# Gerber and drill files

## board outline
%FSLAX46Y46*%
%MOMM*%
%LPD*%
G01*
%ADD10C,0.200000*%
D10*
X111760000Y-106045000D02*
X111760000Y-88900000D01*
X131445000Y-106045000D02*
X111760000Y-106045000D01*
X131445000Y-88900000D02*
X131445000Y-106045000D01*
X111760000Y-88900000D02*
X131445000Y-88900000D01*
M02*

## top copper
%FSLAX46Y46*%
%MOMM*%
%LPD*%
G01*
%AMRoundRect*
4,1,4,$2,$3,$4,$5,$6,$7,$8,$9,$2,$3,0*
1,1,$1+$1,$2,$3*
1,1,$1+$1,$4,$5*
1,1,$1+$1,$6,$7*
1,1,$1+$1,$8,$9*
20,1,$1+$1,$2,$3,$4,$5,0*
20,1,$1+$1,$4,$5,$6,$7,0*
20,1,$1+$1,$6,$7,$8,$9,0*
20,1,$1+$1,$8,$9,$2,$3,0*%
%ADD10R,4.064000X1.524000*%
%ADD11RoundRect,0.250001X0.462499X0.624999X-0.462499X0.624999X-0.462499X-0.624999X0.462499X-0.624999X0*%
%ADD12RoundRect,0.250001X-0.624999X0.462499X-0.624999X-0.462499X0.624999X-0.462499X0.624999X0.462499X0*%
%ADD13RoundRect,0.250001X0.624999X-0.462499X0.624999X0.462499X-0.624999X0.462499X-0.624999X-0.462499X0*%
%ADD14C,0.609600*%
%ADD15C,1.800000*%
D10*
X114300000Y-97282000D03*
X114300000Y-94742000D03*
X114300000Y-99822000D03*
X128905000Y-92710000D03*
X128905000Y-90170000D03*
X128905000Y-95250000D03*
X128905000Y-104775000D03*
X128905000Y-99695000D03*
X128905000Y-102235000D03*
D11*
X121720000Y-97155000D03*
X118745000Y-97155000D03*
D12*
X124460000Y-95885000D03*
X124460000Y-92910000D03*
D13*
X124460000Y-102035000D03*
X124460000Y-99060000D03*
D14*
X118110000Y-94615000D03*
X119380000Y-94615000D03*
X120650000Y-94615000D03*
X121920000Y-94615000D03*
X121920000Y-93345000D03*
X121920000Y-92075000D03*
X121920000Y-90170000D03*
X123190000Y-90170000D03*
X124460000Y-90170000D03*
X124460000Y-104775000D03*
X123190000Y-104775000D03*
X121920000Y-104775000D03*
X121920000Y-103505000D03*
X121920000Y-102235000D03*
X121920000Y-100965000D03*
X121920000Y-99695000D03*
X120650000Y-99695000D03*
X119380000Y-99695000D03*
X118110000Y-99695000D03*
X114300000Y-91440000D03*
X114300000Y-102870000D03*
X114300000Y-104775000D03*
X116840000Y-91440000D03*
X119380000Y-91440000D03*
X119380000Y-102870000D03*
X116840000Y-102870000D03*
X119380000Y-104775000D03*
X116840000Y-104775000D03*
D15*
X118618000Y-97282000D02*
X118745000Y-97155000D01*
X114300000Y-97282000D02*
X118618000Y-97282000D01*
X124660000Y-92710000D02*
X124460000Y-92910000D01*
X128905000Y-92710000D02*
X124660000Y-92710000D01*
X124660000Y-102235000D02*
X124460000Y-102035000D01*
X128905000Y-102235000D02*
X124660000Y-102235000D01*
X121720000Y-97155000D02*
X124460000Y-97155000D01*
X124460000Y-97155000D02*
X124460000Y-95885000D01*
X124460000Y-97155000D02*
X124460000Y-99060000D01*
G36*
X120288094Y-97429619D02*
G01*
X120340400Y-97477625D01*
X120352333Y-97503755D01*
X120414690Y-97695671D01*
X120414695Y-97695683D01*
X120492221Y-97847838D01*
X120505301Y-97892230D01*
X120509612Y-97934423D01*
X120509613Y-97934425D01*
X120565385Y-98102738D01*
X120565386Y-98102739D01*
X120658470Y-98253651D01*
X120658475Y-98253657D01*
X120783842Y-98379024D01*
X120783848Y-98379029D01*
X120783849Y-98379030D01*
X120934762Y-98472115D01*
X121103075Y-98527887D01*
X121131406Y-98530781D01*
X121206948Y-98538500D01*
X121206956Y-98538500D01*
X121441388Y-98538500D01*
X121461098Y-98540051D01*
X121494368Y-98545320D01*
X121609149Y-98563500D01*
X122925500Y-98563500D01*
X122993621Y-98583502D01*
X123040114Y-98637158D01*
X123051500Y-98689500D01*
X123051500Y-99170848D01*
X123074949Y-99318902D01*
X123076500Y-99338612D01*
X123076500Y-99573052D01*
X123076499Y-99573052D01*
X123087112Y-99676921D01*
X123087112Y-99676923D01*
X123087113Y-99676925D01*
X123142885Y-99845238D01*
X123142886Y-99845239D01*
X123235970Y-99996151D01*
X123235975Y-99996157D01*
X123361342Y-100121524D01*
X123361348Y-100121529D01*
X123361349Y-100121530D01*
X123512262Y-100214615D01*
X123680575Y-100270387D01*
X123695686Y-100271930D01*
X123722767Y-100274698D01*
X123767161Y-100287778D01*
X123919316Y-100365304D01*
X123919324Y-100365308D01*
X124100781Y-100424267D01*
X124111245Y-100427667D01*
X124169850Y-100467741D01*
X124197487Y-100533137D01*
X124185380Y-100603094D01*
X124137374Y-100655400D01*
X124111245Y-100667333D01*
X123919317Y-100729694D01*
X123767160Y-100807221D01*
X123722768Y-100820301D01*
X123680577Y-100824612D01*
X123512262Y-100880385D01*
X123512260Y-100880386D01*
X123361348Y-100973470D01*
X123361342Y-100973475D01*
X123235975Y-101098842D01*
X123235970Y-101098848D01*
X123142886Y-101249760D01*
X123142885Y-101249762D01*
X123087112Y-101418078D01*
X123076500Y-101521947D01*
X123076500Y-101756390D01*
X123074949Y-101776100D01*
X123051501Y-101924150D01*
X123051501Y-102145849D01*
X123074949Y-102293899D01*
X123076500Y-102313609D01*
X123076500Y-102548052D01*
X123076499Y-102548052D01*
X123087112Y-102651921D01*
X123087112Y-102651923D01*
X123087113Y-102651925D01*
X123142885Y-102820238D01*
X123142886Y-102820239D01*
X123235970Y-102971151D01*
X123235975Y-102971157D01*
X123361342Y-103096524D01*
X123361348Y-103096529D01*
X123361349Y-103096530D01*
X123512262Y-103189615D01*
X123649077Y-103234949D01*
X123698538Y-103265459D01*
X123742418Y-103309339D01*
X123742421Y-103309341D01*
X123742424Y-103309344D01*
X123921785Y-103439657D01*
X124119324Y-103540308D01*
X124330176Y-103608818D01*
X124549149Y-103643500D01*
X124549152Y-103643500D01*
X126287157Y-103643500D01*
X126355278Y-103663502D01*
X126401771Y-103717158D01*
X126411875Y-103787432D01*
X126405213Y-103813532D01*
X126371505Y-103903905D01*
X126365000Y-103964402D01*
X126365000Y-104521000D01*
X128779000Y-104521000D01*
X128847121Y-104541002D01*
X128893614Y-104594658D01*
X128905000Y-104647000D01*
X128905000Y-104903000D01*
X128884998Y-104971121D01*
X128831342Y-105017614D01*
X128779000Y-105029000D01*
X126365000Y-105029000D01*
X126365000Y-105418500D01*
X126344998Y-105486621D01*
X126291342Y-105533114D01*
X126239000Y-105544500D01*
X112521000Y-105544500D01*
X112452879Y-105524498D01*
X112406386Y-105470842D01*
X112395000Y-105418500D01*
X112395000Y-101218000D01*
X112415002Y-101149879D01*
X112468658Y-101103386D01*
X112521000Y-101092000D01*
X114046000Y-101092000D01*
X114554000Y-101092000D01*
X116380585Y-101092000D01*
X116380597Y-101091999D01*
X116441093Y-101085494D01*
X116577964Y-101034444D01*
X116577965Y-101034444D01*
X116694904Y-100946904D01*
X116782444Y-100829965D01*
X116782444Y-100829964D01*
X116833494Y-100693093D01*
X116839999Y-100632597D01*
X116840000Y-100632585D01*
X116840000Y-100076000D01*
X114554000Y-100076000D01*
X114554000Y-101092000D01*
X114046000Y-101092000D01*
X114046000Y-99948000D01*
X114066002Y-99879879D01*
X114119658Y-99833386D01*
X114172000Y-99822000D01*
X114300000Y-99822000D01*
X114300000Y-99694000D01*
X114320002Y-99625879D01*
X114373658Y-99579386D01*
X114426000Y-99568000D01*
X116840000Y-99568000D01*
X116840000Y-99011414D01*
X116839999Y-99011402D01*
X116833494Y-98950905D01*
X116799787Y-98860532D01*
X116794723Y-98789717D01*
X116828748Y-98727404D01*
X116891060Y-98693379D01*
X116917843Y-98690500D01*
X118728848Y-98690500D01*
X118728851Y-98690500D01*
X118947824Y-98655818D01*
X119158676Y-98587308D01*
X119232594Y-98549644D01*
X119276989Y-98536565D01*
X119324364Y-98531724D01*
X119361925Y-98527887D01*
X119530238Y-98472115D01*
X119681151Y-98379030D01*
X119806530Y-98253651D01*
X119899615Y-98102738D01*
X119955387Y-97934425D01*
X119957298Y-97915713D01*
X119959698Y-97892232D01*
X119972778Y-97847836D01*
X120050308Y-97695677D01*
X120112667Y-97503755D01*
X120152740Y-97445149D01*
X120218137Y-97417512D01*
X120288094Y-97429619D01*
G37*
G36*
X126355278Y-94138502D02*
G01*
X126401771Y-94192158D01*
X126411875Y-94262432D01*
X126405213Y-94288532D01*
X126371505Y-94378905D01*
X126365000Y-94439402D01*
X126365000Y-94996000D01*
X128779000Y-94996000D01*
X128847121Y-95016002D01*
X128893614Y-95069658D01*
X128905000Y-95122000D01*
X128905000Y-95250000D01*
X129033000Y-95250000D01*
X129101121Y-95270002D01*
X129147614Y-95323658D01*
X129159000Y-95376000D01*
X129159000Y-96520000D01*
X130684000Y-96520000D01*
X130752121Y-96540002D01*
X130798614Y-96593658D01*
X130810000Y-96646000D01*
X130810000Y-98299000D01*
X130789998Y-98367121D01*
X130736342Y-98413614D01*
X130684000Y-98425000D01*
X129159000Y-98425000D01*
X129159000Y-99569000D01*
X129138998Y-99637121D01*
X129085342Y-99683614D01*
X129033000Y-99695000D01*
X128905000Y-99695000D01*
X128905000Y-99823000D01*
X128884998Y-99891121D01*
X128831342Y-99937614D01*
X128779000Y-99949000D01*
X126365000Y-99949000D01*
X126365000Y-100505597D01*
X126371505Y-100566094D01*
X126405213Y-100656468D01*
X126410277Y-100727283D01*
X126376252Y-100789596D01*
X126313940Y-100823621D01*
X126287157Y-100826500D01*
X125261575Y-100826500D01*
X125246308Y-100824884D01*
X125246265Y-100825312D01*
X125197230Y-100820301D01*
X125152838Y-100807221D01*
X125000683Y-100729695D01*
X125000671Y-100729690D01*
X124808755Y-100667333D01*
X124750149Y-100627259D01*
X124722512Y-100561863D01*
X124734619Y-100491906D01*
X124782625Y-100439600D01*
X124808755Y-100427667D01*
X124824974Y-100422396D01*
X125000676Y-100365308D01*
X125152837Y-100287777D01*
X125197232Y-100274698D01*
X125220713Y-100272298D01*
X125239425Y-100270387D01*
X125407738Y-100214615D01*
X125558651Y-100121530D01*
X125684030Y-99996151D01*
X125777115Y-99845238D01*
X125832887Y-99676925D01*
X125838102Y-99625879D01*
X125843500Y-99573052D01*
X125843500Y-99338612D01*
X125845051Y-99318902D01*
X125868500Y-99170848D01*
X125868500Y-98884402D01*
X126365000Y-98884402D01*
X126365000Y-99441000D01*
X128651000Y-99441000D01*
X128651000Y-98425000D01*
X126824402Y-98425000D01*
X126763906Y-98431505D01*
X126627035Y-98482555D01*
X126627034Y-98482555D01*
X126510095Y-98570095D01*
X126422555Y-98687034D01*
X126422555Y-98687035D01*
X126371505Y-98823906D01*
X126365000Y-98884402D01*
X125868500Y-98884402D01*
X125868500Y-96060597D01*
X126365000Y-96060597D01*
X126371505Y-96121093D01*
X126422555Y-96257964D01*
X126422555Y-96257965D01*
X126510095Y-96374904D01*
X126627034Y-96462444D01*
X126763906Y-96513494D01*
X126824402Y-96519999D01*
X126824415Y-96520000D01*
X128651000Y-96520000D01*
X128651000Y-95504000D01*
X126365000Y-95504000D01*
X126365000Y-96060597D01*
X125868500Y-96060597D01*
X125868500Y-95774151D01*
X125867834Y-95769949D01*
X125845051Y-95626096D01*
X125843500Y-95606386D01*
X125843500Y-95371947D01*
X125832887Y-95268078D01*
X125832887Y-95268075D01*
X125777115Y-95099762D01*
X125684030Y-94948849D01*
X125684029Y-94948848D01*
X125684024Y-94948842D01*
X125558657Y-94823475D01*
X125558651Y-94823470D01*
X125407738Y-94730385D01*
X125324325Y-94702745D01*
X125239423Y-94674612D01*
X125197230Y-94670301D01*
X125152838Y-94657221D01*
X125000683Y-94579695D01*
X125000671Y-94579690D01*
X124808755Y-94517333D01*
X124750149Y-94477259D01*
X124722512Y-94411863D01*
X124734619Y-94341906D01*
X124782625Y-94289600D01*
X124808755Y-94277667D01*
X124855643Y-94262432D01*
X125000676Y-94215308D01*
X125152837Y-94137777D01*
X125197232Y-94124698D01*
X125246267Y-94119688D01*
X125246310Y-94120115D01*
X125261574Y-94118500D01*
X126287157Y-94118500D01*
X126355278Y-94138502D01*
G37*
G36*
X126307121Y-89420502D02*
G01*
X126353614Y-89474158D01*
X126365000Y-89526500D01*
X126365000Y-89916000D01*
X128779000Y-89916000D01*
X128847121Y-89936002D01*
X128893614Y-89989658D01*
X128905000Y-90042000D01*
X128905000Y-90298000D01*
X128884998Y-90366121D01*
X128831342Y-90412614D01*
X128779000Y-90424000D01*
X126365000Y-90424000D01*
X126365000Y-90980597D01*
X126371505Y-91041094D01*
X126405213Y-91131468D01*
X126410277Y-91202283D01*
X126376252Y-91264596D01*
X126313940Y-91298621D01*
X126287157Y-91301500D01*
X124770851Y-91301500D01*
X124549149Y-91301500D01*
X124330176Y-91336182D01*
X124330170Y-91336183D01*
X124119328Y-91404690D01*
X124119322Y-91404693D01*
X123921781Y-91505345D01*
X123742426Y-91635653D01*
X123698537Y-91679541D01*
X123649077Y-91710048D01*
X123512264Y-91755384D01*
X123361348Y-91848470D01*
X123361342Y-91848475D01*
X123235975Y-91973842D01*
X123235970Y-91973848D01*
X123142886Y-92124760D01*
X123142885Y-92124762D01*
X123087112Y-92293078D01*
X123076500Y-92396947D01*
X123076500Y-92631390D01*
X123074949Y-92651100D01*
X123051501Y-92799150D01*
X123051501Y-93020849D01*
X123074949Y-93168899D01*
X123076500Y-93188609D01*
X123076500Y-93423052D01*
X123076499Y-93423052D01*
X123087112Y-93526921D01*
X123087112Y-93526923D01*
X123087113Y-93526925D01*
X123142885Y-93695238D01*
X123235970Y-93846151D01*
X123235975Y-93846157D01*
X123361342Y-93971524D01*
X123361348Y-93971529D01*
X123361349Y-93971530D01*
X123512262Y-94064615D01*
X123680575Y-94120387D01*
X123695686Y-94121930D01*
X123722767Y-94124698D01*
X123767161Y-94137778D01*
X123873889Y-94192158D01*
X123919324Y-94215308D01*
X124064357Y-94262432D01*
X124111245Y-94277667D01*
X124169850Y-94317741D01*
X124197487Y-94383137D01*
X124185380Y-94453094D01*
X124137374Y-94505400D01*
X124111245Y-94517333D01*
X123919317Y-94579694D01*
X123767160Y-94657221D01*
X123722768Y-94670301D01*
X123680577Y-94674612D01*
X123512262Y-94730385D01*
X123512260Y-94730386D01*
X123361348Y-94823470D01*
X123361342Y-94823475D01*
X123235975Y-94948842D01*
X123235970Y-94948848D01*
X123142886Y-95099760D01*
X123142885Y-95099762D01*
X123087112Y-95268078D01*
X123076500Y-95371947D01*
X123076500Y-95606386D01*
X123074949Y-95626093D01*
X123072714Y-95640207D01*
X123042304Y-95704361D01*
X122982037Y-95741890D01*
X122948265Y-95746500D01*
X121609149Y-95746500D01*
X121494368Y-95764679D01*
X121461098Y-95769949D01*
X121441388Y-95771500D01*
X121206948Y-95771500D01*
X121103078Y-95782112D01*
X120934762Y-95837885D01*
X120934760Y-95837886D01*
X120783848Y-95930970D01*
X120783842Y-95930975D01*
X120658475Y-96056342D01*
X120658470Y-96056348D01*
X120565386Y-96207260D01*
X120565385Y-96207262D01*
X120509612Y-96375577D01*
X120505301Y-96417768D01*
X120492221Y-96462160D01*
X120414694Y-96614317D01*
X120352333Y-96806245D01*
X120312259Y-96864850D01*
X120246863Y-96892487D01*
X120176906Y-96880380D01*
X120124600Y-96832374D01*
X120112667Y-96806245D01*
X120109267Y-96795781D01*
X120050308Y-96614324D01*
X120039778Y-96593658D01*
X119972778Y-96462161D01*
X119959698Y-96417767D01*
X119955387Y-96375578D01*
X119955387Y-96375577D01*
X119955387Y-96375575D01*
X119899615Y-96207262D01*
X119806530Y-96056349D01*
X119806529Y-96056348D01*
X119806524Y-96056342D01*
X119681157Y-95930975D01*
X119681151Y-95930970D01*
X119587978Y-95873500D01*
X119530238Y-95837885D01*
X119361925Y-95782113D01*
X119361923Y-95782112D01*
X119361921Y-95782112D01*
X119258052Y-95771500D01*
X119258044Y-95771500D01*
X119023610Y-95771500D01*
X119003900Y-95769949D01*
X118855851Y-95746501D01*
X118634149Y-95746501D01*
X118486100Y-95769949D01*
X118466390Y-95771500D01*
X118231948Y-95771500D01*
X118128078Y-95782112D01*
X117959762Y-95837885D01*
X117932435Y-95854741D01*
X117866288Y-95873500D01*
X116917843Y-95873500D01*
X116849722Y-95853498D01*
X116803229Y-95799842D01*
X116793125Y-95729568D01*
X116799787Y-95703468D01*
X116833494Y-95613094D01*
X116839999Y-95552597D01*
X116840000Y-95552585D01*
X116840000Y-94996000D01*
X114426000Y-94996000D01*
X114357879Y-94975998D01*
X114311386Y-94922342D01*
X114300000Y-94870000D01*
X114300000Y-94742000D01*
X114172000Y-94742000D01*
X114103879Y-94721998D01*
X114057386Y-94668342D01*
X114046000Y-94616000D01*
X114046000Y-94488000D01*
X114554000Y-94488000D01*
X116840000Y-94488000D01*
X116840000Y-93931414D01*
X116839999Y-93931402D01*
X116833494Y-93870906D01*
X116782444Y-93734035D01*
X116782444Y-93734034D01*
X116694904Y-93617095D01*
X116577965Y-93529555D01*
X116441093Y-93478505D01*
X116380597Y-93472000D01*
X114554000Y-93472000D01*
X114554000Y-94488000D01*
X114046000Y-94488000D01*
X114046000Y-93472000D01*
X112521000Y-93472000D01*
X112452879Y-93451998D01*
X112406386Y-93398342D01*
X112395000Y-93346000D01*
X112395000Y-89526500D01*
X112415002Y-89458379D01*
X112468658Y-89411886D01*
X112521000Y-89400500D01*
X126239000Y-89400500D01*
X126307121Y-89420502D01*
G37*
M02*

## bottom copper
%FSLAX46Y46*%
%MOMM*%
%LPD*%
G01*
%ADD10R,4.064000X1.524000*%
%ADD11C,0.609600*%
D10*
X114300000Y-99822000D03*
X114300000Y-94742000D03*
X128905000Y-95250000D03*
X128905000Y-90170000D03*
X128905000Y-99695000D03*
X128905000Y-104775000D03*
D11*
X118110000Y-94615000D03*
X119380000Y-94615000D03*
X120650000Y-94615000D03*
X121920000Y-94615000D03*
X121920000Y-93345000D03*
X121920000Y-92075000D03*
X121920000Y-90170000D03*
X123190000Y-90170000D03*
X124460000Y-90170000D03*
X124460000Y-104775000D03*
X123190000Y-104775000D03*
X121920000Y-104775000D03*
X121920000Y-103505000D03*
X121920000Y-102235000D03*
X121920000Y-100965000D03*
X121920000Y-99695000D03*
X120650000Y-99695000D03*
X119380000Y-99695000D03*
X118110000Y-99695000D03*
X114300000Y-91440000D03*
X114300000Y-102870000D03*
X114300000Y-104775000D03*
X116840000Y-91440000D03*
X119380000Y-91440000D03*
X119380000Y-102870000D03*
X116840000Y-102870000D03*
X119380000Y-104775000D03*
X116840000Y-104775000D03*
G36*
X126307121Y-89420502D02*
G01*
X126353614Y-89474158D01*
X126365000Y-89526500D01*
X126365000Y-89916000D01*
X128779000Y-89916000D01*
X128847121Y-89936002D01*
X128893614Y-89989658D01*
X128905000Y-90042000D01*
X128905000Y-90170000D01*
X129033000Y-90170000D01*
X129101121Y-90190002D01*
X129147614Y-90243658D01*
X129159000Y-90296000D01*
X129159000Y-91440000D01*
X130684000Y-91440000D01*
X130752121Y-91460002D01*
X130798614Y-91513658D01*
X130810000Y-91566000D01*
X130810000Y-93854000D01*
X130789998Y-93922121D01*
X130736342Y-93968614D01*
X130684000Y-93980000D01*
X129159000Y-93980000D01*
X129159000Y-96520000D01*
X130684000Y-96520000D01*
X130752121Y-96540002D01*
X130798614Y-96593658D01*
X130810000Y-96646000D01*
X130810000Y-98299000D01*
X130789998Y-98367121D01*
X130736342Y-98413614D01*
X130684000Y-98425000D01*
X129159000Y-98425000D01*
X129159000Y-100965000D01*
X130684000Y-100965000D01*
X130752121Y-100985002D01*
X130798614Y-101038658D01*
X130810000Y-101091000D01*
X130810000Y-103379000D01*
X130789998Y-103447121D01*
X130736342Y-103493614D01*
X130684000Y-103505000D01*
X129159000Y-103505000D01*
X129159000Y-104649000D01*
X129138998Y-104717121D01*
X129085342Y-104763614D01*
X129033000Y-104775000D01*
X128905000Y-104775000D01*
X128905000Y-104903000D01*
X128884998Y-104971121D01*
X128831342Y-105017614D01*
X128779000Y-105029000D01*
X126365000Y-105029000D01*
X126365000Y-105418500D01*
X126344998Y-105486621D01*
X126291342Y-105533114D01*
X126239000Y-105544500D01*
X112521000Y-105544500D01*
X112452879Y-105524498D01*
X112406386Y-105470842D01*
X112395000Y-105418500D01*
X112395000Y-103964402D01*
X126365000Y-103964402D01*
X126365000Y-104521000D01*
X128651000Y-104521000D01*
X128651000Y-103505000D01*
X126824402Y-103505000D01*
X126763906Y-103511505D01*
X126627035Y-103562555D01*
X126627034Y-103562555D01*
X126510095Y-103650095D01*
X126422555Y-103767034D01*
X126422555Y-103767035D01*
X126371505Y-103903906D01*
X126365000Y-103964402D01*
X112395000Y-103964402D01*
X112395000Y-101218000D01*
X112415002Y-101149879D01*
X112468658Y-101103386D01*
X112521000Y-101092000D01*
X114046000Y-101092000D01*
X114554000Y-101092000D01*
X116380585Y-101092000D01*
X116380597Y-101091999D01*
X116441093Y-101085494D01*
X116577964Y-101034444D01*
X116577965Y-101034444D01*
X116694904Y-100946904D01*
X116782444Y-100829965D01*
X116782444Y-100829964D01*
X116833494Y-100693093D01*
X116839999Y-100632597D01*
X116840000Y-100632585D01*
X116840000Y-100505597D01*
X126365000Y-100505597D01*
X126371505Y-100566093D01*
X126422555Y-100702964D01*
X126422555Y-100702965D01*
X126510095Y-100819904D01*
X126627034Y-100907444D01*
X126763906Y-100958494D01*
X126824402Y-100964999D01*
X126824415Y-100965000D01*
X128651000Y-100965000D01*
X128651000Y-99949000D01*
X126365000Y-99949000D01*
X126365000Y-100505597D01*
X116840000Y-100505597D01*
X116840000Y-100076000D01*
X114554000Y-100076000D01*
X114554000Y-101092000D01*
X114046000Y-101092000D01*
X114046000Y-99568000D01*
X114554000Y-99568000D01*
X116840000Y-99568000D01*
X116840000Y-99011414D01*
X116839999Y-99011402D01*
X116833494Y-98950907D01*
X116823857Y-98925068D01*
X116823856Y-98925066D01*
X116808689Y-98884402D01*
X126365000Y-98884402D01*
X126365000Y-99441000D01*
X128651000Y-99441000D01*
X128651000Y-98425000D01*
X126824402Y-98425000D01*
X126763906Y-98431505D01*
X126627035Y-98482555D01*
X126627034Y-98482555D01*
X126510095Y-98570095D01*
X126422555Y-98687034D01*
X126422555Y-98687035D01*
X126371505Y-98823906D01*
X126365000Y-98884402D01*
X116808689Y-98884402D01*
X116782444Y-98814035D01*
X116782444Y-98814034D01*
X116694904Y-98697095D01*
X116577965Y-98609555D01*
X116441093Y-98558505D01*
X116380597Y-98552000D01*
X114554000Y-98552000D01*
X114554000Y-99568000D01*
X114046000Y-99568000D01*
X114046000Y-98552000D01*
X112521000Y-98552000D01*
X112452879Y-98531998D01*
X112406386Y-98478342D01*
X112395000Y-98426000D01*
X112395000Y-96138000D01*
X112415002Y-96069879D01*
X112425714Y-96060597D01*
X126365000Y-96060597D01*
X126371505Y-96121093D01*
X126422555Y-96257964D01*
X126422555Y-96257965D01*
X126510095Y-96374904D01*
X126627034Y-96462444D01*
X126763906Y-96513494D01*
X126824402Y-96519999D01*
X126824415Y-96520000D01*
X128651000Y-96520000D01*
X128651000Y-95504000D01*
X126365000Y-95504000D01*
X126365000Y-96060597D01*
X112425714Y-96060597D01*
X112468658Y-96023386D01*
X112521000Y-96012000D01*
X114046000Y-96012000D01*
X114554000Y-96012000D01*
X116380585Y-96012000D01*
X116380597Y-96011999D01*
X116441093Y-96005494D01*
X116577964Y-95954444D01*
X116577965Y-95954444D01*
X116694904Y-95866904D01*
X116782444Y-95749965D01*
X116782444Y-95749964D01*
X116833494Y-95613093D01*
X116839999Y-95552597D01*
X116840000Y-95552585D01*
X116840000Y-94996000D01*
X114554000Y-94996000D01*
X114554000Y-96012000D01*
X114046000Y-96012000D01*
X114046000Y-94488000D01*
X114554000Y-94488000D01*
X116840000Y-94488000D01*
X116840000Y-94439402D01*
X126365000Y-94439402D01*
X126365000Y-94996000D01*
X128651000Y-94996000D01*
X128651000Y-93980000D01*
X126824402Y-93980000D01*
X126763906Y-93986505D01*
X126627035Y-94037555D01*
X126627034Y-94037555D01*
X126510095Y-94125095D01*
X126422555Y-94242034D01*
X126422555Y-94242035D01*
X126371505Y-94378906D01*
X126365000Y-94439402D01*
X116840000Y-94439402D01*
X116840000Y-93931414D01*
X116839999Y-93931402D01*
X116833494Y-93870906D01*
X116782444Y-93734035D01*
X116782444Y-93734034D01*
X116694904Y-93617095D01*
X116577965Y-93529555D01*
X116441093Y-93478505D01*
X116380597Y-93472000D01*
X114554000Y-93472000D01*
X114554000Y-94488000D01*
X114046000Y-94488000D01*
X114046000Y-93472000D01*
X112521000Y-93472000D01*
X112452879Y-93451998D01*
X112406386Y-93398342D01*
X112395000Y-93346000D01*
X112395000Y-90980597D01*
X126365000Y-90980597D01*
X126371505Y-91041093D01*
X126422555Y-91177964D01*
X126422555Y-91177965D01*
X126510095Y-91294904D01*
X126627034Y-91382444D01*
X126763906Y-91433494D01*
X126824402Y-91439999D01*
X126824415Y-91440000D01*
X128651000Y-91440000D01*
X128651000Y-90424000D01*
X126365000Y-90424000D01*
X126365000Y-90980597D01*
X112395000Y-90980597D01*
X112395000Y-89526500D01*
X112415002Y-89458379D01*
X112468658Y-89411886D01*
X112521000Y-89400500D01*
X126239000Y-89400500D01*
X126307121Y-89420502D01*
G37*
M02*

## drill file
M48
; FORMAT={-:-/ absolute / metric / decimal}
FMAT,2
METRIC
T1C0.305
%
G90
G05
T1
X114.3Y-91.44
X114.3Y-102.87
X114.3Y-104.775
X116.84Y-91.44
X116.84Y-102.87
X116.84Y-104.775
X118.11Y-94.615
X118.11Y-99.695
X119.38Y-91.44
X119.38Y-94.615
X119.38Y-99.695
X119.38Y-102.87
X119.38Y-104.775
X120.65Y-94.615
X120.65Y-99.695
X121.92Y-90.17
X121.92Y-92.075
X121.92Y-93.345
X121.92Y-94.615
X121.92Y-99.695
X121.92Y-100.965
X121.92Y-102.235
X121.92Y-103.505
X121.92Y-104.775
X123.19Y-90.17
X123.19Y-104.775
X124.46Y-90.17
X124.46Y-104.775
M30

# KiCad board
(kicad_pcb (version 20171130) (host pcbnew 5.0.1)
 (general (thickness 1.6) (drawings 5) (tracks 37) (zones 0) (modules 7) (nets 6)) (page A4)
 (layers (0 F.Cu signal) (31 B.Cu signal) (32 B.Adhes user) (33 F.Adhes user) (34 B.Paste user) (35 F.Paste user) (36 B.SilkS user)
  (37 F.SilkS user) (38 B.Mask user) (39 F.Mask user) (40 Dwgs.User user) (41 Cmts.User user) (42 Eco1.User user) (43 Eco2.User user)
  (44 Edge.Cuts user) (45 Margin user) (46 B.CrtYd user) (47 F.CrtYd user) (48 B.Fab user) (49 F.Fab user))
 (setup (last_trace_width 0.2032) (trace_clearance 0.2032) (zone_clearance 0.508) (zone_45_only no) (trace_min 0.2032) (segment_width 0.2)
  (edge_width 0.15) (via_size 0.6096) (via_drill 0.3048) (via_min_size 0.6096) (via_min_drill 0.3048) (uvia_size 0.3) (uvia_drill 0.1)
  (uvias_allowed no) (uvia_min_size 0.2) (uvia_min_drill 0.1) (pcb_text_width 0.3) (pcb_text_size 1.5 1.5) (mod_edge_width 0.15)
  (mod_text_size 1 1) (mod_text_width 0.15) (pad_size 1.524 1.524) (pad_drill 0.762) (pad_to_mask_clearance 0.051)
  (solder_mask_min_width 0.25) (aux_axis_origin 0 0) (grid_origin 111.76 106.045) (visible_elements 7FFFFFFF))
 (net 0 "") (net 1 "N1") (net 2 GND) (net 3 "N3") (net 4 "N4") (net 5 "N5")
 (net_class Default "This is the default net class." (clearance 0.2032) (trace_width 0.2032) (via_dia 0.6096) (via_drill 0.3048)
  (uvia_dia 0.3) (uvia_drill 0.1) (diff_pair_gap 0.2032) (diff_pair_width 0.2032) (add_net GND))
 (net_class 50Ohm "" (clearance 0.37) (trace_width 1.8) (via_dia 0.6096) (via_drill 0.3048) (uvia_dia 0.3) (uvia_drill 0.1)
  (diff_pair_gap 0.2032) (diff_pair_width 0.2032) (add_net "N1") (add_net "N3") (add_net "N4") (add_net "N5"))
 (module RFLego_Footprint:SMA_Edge (layer F.Cu) (at 112.268 97.282)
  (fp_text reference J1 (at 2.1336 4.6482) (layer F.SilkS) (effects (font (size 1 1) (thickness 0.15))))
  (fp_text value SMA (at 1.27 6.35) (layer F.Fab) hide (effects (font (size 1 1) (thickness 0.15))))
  (pad 1 smd rect (at 2.032 0) (size 4.064 1.524) (layers F.Cu F.Mask) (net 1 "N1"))
  (pad 2 smd rect (at 2.032 -2.54) (size 4.064 1.524) (layers F.Cu F.Mask) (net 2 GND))
  (pad 2 smd rect (at 2.032 2.54) (size 4.064 1.524) (layers B.Cu B.Mask) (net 2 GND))
  (pad 2 smd rect (at 2.032 -2.54) (size 4.064 1.524) (layers B.Cu B.Mask) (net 2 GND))
  (pad 2 smd rect (at 2.032 2.54) (size 4.064 1.524) (layers F.Cu F.Mask) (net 2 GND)))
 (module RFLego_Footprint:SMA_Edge (layer F.Cu) (at 126.873 92.71)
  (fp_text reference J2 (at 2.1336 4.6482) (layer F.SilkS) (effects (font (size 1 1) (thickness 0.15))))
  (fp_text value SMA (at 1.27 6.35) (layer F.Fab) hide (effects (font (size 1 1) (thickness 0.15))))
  (pad 1 smd rect (at 2.032 0) (size 4.064 1.524) (layers F.Cu F.Mask) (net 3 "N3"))
  (pad 2 smd rect (at 2.032 -2.54) (size 4.064 1.524) (layers F.Cu F.Mask) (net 2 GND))
  (pad 2 smd rect (at 2.032 2.54) (size 4.064 1.524) (layers B.Cu B.Mask) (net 2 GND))
  (pad 2 smd rect (at 2.032 -2.54) (size 4.064 1.524) (layers B.Cu B.Mask) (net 2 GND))
  (pad 2 smd rect (at 2.032 2.54) (size 4.064 1.524) (layers F.Cu F.Mask) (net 2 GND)))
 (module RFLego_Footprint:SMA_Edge (layer F.Cu) (at 126.873 102.235)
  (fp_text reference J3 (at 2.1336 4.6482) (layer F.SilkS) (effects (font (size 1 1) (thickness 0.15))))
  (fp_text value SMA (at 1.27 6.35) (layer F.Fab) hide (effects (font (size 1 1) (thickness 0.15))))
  (pad 2 smd rect (at 2.032 2.54) (size 4.064 1.524) (layers F.Cu F.Mask) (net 2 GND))
  (pad 2 smd rect (at 2.032 -2.54) (size 4.064 1.524) (layers B.Cu B.Mask) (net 2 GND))
  (pad 2 smd rect (at 2.032 2.54) (size 4.064 1.524) (layers B.Cu B.Mask) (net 2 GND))
  (pad 2 smd rect (at 2.032 -2.54) (size 4.064 1.524) (layers F.Cu F.Mask) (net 2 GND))
  (pad 1 smd rect (at 2.032 0) (size 4.064 1.524) (layers F.Cu F.Mask) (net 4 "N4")))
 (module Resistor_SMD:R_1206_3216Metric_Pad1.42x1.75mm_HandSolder (layer F.Cu) (at 120.2325 97.155 180)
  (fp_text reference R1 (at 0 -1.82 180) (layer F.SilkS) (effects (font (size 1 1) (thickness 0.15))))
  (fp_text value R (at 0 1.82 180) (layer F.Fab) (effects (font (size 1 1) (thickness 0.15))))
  (pad 1 smd roundrect (at -1.4875 0 180) (size 1.425 1.75) (layers F.Cu F.Paste F.Mask) (roundrect_rratio 0.175439) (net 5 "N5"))
  (pad 2 smd roundrect (at 1.4875 0 180) (size 1.425 1.75) (layers F.Cu F.Paste F.Mask) (roundrect_rratio 0.175439) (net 1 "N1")))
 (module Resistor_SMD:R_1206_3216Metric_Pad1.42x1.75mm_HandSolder (layer F.Cu) (at 124.46 94.3975 270)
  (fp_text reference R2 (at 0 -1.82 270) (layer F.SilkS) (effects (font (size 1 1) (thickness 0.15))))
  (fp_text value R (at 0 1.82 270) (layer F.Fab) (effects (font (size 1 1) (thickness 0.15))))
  (pad 2 smd roundrect (at 1.4875 0 270) (size 1.425 1.75) (layers F.Cu F.Paste F.Mask) (roundrect_rratio 0.175439) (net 5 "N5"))
  (pad 1 smd roundrect (at -1.4875 0 270) (size 1.425 1.75) (layers F.Cu F.Paste F.Mask) (roundrect_rratio 0.175439) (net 3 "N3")))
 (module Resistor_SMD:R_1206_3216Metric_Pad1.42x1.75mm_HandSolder (layer F.Cu) (at 124.46 100.5475 90)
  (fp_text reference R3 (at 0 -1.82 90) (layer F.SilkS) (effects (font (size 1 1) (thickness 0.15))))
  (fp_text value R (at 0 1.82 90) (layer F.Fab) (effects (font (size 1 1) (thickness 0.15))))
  (pad 1 smd roundrect (at -1.4875 0 90) (size 1.425 1.75) (layers F.Cu F.Paste F.Mask) (roundrect_rratio 0.175439) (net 4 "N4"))
  (pad 2 smd roundrect (at 1.4875 0 90) (size 1.425 1.75) (layers F.Cu F.Paste F.Mask) (roundrect_rratio 0.175439) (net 5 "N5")))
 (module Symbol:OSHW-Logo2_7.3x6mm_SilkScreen (layer F.Cu) (at 120.015 92.075)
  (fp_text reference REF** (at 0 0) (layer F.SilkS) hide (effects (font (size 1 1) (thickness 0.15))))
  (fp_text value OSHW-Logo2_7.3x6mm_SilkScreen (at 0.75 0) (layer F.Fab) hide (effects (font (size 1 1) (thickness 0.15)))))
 (gr_line (start 111.76 106.045) (end 111.76 88.9) (layer Edge.Cuts) (width 0.2))
 (gr_line (start 131.445 106.045) (end 111.76 106.045) (layer Edge.Cuts) (width 0.2))
 (gr_line (start 131.445 88.9) (end 131.445 106.045) (layer Edge.Cuts) (width 0.2))
 (gr_line (start 111.76 88.9) (end 131.445 88.9) (layer Edge.Cuts) (width 0.2))
 (segment (start 118.618 97.282) (end 118.745 97.155) (width 1.8) (layer F.Cu) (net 1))
 (segment (start 114.3 97.282) (end 118.618 97.282) (width 1.8) (layer F.Cu) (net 1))
 (via (at 118.11 94.615) (size 0.6096) (drill 0.3048) (layers F.Cu B.Cu) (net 2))
 (via (at 119.38 94.615) (size 0.6096) (drill 0.3048) (layers F.Cu B.Cu) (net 2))
 (via (at 120.65 94.615) (size 0.6096) (drill 0.3048) (layers F.Cu B.Cu) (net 2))
 (via (at 121.92 94.615) (size 0.6096) (drill 0.3048) (layers F.Cu B.Cu) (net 2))
 (via (at 121.92 93.345) (size 0.6096) (drill 0.3048) (layers F.Cu B.Cu) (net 2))
 (via (at 121.92 92.075) (size 0.6096) (drill 0.3048) (layers F.Cu B.Cu) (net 2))
 (via (at 121.92 90.17) (size 0.6096) (drill 0.3048) (layers F.Cu B.Cu) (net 2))
 (via (at 123.19 90.17) (size 0.6096) (drill 0.3048) (layers F.Cu B.Cu) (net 2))
 (via (at 124.46 90.17) (size 0.6096) (drill 0.3048) (layers F.Cu B.Cu) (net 2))
 (via (at 124.46 104.775) (size 0.6096) (drill 0.3048) (layers F.Cu B.Cu) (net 2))
 (via (at 123.19 104.775) (size 0.6096) (drill 0.3048) (layers F.Cu B.Cu) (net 2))
 (via (at 121.92 104.775) (size 0.6096) (drill 0.3048) (layers F.Cu B.Cu) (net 2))
 (via (at 121.92 103.505) (size 0.6096) (drill 0.3048) (layers F.Cu B.Cu) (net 2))
 (via (at 121.92 102.235) (size 0.6096) (drill 0.3048) (layers F.Cu B.Cu) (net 2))
 (via (at 121.92 100.965) (size 0.6096) (drill 0.3048) (layers F.Cu B.Cu) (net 2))
 (via (at 121.92 99.695) (size 0.6096) (drill 0.3048) (layers F.Cu B.Cu) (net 2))
 (via (at 120.65 99.695) (size 0.6096) (drill 0.3048) (layers F.Cu B.Cu) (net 2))
 (via (at 119.38 99.695) (size 0.6096) (drill 0.3048) (layers F.Cu B.Cu) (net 2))
 (via (at 118.11 99.695) (size 0.6096) (drill 0.3048) (layers F.Cu B.Cu) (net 2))
 (via (at 114.3 91.44) (size 0.6096) (drill 0.3048) (layers F.Cu B.Cu) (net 2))
 (via (at 114.3 102.87) (size 0.6096) (drill 0.3048) (layers F.Cu B.Cu) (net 2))
 (via (at 114.3 104.775) (size 0.6096) (drill 0.3048) (layers F.Cu B.Cu) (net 2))
 (via (at 116.84 91.44) (size 0.6096) (drill 0.3048) (layers F.Cu B.Cu) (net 2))
 (via (at 119.38 91.44) (size 0.6096) (drill 0.3048) (layers F.Cu B.Cu) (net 2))
 (via (at 119.38 102.87) (size 0.6096) (drill 0.3048) (layers F.Cu B.Cu) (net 2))
 (via (at 116.84 102.87) (size 0.6096) (drill 0.3048) (layers F.Cu B.Cu) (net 2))
 (via (at 119.38 104.775) (size 0.6096) (drill 0.3048) (layers F.Cu B.Cu) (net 2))
 (via (at 116.84 104.775) (size 0.6096) (drill 0.3048) (layers F.Cu B.Cu) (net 2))
 (segment (start 124.66 92.71) (end 124.46 92.91) (width 1.8) (layer F.Cu) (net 3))
 (segment (start 128.905 92.71) (end 124.66 92.71) (width 1.8) (layer F.Cu) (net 3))
 (segment (start 124.66 102.235) (end 124.46 102.035) (width 1.8) (layer F.Cu) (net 4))
 (segment (start 128.905 102.235) (end 124.66 102.235) (width 1.8) (layer F.Cu) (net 4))
 (segment (start 121.72 97.155) (end 124.46 97.155) (width 1.8) (layer F.Cu) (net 5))
 (segment (start 124.46 97.155) (end 124.46 95.885) (width 1.8) (layer F.Cu) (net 5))
 (segment (start 124.46 97.155) (end 124.46 99.06) (width 1.8) (layer F.Cu) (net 5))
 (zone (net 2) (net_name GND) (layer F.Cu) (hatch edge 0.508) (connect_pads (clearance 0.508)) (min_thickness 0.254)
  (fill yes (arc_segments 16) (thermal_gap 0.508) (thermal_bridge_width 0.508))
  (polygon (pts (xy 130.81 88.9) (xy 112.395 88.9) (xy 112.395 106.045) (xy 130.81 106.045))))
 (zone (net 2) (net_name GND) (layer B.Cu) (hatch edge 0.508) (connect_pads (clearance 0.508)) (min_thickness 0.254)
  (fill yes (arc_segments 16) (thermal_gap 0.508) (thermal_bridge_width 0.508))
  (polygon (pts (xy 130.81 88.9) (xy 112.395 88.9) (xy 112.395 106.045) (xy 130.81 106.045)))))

